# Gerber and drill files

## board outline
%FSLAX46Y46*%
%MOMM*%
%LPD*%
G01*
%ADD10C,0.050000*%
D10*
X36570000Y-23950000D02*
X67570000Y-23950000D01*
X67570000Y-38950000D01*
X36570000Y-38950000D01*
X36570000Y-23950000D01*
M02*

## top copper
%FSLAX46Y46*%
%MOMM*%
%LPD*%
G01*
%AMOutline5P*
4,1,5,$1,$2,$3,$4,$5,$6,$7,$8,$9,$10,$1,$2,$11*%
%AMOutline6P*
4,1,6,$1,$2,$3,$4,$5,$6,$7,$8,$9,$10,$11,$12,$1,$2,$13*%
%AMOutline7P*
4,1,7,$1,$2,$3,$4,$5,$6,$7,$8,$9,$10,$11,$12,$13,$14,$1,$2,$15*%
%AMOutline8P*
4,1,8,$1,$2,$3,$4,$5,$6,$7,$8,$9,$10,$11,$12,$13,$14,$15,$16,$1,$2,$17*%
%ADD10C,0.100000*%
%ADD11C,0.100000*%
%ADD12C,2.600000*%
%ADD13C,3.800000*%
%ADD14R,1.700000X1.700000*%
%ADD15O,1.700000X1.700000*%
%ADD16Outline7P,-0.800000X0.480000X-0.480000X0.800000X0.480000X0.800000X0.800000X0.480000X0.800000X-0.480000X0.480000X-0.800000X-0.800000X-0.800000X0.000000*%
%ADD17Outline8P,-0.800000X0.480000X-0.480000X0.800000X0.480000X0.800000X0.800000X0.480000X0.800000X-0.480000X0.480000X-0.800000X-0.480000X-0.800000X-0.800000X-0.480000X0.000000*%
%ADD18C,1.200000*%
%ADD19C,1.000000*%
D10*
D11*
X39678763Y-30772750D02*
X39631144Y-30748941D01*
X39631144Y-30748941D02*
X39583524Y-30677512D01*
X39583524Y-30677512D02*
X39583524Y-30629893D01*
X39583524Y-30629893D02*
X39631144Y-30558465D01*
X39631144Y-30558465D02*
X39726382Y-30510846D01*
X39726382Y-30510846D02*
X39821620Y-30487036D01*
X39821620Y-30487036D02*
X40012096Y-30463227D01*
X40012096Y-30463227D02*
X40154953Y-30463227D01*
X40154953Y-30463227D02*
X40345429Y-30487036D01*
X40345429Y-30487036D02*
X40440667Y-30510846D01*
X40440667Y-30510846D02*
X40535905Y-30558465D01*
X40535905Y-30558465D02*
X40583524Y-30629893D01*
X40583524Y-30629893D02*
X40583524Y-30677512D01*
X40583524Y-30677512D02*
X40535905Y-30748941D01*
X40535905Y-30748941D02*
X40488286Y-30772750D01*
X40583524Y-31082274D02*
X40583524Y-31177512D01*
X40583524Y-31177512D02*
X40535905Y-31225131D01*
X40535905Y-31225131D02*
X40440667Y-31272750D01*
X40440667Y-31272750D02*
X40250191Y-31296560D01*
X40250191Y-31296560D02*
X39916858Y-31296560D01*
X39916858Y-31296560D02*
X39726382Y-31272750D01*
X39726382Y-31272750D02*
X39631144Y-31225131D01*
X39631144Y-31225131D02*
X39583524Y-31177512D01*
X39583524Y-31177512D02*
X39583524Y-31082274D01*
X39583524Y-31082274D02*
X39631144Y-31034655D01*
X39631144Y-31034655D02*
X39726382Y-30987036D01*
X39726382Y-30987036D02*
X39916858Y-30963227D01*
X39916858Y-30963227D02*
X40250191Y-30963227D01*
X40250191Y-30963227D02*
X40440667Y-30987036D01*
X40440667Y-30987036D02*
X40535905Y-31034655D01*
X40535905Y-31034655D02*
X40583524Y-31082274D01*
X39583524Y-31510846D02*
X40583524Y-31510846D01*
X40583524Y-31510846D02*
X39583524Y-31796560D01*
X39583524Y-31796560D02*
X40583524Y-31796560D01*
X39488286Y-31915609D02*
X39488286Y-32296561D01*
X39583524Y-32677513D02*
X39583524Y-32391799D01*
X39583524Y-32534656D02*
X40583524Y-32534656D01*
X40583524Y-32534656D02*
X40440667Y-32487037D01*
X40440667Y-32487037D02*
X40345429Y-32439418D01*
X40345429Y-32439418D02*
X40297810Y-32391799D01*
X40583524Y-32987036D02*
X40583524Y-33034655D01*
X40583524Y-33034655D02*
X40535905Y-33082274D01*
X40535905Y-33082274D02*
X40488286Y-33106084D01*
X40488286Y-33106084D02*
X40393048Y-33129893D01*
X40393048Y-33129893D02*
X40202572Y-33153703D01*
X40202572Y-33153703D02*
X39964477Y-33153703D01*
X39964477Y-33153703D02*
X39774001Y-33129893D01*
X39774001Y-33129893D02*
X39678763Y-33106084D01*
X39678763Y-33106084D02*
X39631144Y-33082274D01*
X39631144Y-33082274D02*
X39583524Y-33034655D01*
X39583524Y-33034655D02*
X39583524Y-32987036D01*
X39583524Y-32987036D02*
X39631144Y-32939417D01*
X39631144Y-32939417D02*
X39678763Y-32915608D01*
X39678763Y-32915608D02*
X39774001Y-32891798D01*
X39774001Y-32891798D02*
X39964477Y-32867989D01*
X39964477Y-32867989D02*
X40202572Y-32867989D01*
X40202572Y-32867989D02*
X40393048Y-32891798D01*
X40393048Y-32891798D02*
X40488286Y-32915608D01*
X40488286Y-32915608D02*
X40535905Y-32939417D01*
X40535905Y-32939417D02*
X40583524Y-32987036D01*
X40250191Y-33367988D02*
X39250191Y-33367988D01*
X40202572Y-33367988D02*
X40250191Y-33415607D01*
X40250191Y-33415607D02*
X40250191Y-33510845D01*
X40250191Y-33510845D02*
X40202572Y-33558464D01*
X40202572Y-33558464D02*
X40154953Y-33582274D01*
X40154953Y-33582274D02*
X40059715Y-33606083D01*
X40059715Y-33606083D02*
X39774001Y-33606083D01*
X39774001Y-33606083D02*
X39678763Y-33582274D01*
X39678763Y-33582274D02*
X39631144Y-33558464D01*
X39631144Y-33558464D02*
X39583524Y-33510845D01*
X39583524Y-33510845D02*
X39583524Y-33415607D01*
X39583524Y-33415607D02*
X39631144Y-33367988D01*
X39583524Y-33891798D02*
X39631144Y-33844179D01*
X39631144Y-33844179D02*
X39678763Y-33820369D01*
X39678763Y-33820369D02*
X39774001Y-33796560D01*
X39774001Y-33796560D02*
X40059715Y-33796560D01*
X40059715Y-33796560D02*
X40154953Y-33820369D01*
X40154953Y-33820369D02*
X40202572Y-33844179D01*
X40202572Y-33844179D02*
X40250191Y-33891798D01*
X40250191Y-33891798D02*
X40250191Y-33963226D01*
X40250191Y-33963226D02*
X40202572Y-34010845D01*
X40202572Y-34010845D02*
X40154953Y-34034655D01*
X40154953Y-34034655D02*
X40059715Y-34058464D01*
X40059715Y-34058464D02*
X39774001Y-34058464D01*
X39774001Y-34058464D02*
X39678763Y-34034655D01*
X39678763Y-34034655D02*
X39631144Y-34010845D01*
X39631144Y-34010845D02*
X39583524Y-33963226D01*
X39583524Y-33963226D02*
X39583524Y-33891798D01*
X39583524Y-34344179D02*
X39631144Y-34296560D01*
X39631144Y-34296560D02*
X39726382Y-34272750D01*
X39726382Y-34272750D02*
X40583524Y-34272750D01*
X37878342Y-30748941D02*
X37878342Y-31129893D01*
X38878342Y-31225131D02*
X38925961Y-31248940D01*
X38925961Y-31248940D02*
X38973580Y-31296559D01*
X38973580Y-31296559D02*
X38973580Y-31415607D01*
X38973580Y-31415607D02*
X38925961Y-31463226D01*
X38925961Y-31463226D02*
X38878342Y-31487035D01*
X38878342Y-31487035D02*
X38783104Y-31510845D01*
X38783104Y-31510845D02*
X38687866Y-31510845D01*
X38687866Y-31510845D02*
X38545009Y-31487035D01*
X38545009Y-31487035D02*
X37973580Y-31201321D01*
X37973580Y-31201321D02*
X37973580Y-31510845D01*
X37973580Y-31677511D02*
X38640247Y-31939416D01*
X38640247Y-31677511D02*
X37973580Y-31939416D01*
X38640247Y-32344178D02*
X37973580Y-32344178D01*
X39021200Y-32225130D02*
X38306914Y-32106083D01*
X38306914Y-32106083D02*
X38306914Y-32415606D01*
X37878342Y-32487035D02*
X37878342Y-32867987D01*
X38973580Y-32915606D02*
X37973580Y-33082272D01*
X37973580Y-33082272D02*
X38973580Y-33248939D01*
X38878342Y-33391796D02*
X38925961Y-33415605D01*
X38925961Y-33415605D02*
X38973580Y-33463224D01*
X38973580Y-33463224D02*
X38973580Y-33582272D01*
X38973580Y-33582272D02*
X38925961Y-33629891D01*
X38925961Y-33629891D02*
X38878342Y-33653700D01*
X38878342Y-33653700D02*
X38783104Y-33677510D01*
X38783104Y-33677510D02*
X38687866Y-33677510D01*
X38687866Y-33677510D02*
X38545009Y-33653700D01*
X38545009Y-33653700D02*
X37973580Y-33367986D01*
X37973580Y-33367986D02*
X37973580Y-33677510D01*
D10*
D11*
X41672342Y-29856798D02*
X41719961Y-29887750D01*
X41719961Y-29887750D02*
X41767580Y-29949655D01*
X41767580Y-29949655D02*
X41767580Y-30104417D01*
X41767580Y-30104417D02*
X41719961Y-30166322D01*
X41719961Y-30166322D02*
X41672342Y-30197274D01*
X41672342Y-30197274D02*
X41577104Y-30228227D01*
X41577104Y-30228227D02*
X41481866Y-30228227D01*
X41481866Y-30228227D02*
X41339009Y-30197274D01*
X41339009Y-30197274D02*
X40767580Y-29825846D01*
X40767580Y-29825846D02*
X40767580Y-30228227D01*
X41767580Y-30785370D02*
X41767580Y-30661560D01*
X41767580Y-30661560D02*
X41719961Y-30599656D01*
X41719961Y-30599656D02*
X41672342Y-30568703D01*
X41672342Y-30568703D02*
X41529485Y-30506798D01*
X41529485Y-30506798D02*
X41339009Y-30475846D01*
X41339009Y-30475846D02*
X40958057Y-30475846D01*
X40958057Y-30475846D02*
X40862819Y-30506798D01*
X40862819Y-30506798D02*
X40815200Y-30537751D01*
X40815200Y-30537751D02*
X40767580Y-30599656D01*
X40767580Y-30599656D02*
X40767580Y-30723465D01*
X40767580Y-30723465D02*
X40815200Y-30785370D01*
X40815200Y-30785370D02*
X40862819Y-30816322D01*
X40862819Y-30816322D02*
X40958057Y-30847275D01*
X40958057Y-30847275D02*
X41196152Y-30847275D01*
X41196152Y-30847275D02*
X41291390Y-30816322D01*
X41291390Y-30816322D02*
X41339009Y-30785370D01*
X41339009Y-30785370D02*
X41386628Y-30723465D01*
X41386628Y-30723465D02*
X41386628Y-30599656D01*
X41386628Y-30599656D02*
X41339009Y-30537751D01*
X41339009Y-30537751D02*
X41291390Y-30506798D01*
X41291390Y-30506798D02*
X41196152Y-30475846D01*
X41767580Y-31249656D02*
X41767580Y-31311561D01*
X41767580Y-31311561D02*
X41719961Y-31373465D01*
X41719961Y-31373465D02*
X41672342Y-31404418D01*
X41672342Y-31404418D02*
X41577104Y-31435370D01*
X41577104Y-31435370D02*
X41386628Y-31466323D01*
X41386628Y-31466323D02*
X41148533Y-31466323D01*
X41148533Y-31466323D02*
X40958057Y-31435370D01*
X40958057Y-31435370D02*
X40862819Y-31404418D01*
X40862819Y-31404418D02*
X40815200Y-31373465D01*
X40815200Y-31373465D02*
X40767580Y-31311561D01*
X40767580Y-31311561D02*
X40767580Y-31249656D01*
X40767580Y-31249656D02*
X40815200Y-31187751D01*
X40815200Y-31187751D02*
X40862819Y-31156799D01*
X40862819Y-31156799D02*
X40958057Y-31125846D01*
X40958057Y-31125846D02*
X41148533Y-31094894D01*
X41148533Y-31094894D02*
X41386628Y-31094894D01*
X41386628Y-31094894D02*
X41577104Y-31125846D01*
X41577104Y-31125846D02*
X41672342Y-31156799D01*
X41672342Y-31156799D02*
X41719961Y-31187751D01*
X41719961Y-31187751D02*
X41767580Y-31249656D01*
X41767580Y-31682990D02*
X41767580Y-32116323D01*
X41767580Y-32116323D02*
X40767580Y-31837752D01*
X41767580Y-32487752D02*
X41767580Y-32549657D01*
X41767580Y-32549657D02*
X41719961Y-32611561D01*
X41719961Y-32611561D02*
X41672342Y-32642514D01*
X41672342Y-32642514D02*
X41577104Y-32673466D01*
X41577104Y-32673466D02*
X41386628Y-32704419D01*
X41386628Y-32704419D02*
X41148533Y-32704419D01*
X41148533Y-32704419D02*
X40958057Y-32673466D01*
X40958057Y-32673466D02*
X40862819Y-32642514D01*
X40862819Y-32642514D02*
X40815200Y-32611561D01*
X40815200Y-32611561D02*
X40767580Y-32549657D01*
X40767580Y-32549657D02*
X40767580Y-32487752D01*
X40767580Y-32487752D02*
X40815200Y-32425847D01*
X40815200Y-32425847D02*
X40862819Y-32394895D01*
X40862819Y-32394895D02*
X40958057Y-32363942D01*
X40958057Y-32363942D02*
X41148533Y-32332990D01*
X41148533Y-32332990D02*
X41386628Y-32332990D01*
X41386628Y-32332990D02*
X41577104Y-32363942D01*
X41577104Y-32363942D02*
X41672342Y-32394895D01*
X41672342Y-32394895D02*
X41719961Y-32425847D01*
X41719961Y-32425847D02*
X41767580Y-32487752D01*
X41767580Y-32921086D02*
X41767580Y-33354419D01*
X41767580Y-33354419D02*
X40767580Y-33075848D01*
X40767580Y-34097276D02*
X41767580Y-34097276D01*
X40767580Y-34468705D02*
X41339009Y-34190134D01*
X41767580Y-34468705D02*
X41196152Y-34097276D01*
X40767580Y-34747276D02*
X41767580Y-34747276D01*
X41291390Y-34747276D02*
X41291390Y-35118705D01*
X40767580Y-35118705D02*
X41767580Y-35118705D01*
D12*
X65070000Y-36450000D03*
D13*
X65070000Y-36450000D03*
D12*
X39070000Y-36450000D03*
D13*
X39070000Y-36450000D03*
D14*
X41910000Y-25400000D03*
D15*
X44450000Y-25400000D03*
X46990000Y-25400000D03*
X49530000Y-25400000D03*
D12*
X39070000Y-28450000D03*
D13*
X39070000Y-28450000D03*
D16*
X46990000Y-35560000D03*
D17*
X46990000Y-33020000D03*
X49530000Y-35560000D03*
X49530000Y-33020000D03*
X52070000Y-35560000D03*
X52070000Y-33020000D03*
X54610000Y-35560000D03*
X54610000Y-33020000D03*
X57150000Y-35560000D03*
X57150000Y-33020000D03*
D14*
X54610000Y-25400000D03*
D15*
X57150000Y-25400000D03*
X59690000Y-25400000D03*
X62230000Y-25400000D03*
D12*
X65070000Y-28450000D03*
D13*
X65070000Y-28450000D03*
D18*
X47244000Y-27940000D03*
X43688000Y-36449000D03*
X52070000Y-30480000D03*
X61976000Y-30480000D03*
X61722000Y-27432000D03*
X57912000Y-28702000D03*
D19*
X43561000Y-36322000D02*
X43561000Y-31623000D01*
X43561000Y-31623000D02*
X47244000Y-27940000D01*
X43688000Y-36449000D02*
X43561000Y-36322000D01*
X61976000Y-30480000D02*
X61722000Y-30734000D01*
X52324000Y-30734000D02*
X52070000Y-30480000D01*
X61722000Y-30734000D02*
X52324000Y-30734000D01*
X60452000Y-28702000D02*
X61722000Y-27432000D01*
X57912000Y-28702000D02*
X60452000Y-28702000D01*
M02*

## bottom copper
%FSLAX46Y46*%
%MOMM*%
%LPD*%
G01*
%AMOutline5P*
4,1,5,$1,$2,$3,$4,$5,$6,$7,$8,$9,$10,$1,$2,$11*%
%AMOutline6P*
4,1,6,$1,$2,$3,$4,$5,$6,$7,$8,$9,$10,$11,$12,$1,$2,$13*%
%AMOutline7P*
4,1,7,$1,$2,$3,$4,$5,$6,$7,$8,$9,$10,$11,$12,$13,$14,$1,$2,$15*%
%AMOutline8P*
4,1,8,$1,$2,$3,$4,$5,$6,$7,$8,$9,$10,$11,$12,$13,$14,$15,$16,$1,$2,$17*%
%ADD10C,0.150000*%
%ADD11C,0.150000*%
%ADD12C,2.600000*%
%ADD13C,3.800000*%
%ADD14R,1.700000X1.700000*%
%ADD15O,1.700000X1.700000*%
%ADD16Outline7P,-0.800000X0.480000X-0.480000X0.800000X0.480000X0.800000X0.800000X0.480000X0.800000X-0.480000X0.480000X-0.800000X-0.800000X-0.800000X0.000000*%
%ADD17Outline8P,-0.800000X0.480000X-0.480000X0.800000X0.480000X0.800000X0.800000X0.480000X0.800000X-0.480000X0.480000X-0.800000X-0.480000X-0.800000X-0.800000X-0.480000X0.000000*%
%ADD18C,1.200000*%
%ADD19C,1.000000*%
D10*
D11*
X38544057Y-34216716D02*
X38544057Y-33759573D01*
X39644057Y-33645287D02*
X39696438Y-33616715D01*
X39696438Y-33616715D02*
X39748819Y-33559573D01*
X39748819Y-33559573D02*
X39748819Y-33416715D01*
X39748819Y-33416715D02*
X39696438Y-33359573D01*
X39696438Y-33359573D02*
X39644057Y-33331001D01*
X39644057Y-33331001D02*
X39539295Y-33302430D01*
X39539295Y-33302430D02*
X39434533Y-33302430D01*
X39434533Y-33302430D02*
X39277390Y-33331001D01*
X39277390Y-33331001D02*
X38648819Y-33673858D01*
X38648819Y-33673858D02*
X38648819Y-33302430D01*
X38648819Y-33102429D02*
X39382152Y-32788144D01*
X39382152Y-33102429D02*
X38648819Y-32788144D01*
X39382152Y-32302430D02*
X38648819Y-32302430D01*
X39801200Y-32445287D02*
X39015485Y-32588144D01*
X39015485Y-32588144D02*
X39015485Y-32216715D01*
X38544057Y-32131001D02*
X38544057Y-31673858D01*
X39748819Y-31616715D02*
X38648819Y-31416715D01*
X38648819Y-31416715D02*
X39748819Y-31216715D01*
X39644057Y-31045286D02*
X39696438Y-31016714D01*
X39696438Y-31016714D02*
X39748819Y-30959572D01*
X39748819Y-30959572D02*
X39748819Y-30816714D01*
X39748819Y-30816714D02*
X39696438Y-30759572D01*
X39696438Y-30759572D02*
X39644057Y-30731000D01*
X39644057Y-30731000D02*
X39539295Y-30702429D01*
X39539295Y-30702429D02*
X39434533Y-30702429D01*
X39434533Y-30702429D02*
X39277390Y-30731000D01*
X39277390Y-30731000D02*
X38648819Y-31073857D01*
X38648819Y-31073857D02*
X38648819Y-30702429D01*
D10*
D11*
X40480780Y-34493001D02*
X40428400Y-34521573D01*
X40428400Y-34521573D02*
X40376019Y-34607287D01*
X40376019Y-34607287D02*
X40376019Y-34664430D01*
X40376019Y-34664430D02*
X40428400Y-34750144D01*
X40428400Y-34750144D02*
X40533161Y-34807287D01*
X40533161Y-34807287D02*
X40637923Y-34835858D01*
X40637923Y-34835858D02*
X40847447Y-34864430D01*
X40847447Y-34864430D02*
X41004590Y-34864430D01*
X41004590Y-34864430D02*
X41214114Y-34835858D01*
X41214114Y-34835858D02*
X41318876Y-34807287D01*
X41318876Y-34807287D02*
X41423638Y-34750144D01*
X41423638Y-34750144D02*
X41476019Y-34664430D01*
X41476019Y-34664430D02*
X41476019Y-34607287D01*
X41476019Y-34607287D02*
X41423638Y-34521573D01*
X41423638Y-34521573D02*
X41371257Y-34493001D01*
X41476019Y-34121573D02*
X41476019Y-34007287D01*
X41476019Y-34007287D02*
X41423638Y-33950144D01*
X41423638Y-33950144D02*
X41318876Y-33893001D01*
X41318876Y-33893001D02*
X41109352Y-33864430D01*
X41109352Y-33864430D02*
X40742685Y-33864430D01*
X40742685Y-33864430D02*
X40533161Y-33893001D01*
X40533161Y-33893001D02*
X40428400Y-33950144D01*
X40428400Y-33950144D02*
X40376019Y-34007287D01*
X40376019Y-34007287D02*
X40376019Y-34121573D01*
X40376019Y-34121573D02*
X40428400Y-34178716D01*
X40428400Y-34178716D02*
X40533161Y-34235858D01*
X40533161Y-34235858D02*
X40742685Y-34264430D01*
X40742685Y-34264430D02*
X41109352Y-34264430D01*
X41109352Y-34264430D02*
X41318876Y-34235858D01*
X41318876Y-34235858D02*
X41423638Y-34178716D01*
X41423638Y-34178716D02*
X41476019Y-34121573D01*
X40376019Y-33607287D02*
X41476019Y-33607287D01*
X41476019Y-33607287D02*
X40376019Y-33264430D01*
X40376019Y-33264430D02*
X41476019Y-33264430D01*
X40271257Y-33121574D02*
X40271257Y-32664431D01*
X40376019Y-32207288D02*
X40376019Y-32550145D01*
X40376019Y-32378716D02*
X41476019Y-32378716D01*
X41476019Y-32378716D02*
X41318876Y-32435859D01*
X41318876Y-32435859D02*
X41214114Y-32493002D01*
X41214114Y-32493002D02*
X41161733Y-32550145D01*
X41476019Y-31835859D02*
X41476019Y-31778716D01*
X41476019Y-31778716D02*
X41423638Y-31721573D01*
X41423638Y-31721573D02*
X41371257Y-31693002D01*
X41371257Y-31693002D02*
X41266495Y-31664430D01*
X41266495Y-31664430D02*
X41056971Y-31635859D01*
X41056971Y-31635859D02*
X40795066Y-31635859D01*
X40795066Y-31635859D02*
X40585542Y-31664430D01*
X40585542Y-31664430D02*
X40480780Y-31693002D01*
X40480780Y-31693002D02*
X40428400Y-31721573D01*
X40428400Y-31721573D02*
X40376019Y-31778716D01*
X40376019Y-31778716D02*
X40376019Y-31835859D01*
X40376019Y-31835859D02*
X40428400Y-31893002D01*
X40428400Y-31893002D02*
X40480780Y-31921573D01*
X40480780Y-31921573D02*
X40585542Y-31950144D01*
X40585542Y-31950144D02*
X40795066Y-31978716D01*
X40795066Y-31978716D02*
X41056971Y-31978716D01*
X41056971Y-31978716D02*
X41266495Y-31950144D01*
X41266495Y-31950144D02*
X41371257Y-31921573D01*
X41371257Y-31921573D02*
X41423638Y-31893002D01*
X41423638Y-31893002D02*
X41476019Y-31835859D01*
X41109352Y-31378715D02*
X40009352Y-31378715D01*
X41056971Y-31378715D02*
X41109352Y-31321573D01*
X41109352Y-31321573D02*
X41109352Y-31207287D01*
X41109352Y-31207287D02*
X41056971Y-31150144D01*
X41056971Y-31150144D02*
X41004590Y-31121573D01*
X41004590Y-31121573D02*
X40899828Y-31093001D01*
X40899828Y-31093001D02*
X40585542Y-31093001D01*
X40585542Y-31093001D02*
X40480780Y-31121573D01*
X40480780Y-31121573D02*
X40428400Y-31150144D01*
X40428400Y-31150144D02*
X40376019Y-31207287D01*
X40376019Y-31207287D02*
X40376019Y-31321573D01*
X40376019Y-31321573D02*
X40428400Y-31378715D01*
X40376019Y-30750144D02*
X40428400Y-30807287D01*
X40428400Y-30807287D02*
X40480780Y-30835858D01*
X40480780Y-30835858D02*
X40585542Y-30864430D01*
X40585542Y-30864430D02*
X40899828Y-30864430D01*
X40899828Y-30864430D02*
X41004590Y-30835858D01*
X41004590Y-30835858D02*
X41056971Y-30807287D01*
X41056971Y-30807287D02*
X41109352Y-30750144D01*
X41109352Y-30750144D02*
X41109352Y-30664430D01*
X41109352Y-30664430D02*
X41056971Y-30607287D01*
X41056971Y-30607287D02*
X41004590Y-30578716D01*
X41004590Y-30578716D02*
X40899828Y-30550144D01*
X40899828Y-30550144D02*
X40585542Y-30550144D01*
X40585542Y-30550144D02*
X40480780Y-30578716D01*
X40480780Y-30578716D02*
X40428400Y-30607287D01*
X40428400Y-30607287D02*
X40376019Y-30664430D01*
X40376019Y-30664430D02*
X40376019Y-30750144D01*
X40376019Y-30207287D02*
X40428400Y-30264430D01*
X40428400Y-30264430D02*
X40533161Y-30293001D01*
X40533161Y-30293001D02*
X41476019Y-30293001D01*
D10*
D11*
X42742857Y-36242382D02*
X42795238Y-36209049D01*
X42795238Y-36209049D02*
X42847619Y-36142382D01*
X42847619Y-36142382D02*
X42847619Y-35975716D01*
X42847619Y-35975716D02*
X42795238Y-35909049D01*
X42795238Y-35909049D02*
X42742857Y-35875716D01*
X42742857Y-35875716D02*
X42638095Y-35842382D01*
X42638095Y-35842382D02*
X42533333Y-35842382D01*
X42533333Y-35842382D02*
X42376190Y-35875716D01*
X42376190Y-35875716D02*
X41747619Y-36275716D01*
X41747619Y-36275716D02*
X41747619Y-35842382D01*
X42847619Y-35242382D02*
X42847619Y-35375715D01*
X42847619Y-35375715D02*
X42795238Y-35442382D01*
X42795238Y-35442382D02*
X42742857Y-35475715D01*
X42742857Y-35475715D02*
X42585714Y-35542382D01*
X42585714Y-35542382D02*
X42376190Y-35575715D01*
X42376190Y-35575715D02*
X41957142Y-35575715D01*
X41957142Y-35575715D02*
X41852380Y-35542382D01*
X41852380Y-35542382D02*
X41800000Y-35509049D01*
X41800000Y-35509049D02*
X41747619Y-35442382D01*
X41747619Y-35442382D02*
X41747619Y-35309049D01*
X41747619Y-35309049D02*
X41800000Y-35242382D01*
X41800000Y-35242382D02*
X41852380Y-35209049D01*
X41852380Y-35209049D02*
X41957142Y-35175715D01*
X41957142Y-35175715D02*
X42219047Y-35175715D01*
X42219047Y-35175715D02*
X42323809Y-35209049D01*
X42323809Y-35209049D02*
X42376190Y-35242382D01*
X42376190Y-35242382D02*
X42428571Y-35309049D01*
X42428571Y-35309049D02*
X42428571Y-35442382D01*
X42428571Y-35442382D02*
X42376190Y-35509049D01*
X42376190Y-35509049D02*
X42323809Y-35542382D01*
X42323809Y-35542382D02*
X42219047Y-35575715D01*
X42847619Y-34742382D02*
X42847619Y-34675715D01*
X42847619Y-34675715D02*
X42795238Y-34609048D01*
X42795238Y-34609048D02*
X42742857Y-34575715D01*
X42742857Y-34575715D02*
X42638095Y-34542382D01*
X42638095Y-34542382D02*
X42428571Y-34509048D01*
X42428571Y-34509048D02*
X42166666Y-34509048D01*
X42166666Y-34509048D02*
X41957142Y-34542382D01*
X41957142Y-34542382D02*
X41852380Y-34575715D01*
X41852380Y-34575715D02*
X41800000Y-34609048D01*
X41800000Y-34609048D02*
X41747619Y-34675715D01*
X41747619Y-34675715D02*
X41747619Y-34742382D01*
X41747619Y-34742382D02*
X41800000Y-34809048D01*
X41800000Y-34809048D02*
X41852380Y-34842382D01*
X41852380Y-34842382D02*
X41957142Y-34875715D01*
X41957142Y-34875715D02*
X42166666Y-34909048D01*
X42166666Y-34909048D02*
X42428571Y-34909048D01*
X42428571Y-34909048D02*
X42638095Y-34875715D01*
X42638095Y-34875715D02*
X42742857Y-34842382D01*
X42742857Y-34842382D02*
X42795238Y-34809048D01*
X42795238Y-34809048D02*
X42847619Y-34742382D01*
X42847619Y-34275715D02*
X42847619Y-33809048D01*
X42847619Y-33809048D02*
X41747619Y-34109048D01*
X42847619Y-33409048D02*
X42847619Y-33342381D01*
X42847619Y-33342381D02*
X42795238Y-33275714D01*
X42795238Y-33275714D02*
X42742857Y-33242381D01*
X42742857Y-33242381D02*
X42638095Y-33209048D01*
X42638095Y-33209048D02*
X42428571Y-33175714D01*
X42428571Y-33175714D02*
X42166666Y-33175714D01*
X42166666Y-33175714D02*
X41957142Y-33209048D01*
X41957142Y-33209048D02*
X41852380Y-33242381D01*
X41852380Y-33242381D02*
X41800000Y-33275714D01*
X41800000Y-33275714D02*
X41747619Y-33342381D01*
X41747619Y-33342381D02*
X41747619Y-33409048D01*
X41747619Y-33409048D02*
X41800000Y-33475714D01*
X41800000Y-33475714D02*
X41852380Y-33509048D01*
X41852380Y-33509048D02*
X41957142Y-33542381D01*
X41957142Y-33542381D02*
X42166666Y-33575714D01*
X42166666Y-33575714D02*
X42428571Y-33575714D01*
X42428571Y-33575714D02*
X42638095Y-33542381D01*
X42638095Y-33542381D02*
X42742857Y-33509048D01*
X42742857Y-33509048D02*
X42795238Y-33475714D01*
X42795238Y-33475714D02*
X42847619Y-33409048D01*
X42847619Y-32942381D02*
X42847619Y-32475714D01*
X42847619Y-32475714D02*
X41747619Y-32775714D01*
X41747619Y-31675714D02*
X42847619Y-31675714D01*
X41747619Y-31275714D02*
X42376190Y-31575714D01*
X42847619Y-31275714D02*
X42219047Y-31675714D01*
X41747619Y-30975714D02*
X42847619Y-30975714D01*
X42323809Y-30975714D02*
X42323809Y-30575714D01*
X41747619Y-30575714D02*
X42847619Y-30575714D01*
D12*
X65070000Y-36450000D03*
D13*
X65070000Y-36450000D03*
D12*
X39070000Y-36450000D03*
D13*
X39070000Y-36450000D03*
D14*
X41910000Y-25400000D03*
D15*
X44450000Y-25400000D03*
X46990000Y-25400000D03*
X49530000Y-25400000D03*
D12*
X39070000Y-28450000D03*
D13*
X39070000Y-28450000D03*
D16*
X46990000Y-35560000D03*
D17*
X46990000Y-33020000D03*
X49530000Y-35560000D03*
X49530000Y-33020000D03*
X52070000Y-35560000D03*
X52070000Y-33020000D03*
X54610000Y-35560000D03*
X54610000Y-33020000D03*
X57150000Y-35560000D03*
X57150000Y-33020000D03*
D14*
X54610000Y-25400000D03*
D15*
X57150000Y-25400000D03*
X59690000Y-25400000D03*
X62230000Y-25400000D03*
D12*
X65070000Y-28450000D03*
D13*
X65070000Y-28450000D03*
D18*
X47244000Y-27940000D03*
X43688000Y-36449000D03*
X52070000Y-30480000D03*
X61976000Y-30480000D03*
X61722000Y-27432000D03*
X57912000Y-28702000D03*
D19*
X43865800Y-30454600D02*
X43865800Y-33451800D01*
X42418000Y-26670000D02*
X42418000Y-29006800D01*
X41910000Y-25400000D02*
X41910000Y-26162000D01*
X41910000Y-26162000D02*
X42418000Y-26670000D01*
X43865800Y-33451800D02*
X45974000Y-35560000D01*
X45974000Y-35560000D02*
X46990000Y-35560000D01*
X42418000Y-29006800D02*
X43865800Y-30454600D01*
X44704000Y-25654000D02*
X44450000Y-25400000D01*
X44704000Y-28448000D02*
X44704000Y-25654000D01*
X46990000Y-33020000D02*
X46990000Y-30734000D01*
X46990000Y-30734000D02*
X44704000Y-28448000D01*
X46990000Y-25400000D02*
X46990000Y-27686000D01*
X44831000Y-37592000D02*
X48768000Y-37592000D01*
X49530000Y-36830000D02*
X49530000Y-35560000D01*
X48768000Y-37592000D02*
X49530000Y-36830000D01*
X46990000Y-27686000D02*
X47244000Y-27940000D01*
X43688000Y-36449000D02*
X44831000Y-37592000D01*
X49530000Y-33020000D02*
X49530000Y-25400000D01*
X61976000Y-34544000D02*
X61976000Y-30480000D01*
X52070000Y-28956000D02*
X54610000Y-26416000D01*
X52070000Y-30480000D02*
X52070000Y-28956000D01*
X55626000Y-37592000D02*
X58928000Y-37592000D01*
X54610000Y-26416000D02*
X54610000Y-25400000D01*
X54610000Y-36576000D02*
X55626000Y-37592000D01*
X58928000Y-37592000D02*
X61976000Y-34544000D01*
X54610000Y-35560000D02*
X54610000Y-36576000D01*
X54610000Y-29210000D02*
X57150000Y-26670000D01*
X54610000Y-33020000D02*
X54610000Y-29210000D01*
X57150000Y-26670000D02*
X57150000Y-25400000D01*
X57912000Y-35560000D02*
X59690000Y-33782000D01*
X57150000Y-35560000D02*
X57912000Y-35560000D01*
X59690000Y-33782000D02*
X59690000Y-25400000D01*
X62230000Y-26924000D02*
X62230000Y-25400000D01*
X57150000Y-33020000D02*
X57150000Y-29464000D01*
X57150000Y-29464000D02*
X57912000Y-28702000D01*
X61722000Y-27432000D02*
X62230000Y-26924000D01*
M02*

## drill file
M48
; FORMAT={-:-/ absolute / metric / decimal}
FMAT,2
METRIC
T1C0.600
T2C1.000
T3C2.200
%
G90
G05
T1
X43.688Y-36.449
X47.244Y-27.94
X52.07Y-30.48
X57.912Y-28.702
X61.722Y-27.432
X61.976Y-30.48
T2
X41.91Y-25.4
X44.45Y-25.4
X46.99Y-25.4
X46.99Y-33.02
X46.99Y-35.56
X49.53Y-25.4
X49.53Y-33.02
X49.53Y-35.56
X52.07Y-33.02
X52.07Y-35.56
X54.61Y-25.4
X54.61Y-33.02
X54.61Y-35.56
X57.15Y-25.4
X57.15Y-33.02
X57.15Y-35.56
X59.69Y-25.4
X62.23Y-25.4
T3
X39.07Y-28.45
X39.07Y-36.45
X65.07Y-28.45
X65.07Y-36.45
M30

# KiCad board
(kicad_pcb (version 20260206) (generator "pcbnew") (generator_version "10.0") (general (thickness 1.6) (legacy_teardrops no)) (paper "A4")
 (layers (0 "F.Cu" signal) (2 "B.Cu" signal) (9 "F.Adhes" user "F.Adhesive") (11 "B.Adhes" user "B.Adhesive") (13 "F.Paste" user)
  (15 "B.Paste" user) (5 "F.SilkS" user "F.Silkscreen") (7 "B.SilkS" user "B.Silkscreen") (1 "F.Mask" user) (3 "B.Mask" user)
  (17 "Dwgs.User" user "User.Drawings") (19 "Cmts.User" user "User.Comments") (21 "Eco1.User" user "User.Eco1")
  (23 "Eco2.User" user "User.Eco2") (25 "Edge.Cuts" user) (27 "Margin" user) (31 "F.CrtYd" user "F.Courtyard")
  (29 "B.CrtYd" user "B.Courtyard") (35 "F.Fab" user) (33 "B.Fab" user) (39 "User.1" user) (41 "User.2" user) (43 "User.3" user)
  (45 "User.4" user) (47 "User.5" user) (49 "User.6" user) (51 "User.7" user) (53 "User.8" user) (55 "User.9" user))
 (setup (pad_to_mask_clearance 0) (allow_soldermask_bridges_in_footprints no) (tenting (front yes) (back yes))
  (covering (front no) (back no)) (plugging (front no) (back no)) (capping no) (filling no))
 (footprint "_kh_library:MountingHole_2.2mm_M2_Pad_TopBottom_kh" (layer "F.Cu") (at 65.07 36.45)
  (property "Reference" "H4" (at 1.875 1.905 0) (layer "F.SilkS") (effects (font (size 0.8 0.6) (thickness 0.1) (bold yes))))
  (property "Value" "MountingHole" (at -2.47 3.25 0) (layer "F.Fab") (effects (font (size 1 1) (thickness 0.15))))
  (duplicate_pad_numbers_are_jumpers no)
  (pad "1" thru_hole circle (at 0 0) (size 2.6 2.6) (drill 2.2) (layers "*.Cu" "*.Mask") (remove_unused_layers no))
  (pad "1" connect circle (at 0 0) (size 3.8 3.8) (layers "F.Cu" "F.Mask"))
  (pad "1" connect circle (at 0 0) (size 3.8 3.8) (layers "B.Cu" "B.Mask")))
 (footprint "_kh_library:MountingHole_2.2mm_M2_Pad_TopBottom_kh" (layer "F.Cu") (at 39.07 36.45)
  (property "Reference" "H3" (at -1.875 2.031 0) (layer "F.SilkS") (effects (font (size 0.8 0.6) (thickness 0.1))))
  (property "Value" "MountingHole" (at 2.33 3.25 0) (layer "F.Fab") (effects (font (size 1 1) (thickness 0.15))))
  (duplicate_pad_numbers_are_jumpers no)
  (pad "1" thru_hole circle (at 0 0) (size 2.6 2.6) (drill 2.2) (layers "*.Cu" "*.Mask") (remove_unused_layers no))
  (pad "1" connect circle (at 0 0) (size 3.8 3.8) (layers "F.Cu" "F.Mask"))
  (pad "1" connect circle (at 0 0) (size 3.8 3.8) (layers "B.Cu" "B.Mask")))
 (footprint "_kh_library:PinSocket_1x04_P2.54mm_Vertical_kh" (layer "F.Cu") (at 41.91 25.4 90)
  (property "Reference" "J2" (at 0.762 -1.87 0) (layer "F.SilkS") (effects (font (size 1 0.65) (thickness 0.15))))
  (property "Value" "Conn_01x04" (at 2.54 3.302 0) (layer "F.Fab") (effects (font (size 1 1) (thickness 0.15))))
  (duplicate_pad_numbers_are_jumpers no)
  (pad "1" thru_hole rect (at 0 0 90) (size 1.7 1.7) (drill 1) (layers "*.Cu" "*.Mask") (remove_unused_layers no) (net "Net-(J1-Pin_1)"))
  (pad "2" thru_hole oval (at 0 2.54 90) (size 1.7 1.7) (drill 1) (layers "*.Cu" "*.Mask") (remove_unused_layers no) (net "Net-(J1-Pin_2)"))
  (pad "3" thru_hole oval (at 0 5.08 90) (size 1.7 1.7) (drill 1) (layers "*.Cu" "*.Mask") (remove_unused_layers no) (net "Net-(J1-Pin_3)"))
  (pad "4" thru_hole oval (at 0 7.62 90) (size 1.7 1.7) (drill 1) (layers "*.Cu" "*.Mask") (remove_unused_layers no) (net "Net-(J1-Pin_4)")))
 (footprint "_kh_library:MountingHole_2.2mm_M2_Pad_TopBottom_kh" (layer "F.Cu") (at 39.07 28.45)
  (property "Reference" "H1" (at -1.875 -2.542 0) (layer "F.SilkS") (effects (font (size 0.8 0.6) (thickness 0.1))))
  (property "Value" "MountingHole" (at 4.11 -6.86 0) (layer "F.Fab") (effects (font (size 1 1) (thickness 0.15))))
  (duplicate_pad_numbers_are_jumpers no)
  (pad "1" thru_hole circle (at 0 0) (size 2.6 2.6) (drill 2.2) (layers "*.Cu" "*.Mask") (remove_unused_layers no))
  (pad "1" connect circle (at 0 0) (size 3.8 3.8) (layers "F.Cu" "F.Mask"))
  (pad "1" connect circle (at 0 0) (size 3.8 3.8) (layers "B.Cu" "B.Mask")))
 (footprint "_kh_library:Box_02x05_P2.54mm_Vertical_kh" (layer "F.Cu") (at 46.99 35.56)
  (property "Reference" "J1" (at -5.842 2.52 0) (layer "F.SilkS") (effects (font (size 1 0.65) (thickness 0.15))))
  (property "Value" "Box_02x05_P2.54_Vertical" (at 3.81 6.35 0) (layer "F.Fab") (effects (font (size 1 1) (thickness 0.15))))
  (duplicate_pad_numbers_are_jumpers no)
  (pad "1" thru_hole roundrect (at 0 0) (size 1.6 1.6) (drill 1) (layers "*.Cu" "*.Mask") (remove_unused_layers no) (roundrect_rratio 0)
   (chamfer_ratio 0.2) (chamfer top_left top_right bottom_right) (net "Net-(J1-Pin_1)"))
  (pad "2" thru_hole roundrect (at 0 -2.54) (size 1.6 1.6) (drill 1) (layers "*.Cu" "*.Mask") (remove_unused_layers no) (roundrect_rratio 0)
   (chamfer_ratio 0.2) (chamfer top_left top_right bottom_left bottom_right) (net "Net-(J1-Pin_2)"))
  (pad "3" thru_hole roundrect (at 2.54 0) (size 1.6 1.6) (drill 1) (layers "*.Cu" "*.Mask") (remove_unused_layers no) (roundrect_rratio 0)
   (chamfer_ratio 0.2) (chamfer top_left top_right bottom_left bottom_right) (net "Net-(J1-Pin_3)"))
  (pad "4" thru_hole roundrect (at 2.54 -2.54) (size 1.6 1.6) (drill 1) (layers "*.Cu" "*.Mask") (remove_unused_layers no)
   (roundrect_rratio 0) (chamfer_ratio 0.2) (chamfer top_left top_right bottom_left bottom_right) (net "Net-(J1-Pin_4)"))
  (pad "5" thru_hole roundrect (at 5.08 0) (size 1.6 1.6) (drill 1) (layers "*.Cu" "*.Mask") (remove_unused_layers no) (roundrect_rratio 0)
   (chamfer_ratio 0.2) (chamfer top_left top_right bottom_left bottom_right) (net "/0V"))
  (pad "6" thru_hole roundrect (at 5.08 -2.54) (size 1.6 1.6) (drill 1) (layers "*.Cu" "*.Mask") (remove_unused_layers no)
   (roundrect_rratio 0) (chamfer_ratio 0.2) (chamfer top_left top_right bottom_left bottom_right) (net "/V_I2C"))
  (pad "7" thru_hole roundrect (at 7.62 0) (size 1.6 1.6) (drill 1) (layers "*.Cu" "*.Mask") (remove_unused_layers no) (roundrect_rratio 0)
   (chamfer_ratio 0.2) (chamfer top_left top_right bottom_left bottom_right) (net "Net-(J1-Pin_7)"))
  (pad "8" thru_hole roundrect (at 7.62 -2.54) (size 1.6 1.6) (drill 1) (layers "*.Cu" "*.Mask") (remove_unused_layers no)
   (roundrect_rratio 0) (chamfer_ratio 0.2) (chamfer top_left top_right bottom_left bottom_right) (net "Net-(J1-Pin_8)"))
  (pad "9" thru_hole roundrect (at 10.16 0) (size 1.6 1.6) (drill 1) (layers "*.Cu" "*.Mask") (remove_unused_layers no) (roundrect_rratio 0)
   (chamfer_ratio 0.2) (chamfer top_left top_right bottom_left bottom_right) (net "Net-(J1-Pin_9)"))
  (pad "10" thru_hole roundrect (at 10.16 -2.54) (size 1.6 1.6) (drill 1) (layers "*.Cu" "*.Mask") (remove_unused_layers no)
   (roundrect_rratio 0) (chamfer_ratio 0.2) (chamfer top_left top_right bottom_left bottom_right) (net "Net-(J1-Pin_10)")))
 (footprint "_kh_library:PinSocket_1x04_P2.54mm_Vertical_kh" (layer "F.Cu") (at 54.61 25.4 90)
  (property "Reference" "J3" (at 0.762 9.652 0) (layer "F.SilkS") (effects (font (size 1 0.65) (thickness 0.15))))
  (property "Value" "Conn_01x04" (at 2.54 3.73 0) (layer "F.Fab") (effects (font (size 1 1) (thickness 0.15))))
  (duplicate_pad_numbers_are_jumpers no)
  (pad "1" thru_hole rect (at 0 0 90) (size 1.7 1.7) (drill 1) (layers "*.Cu" "*.Mask") (remove_unused_layers no) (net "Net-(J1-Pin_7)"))
  (pad "2" thru_hole oval (at 0 2.54 90) (size 1.7 1.7) (drill 1) (layers "*.Cu" "*.Mask") (remove_unused_layers no) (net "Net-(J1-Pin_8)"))
  (pad "3" thru_hole oval (at 0 5.08 90) (size 1.7 1.7) (drill 1) (layers "*.Cu" "*.Mask") (remove_unused_layers no) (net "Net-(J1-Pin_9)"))
  (pad "4" thru_hole oval (at 0 7.62 90) (size 1.7 1.7) (drill 1) (layers "*.Cu" "*.Mask") (remove_unused_layers no) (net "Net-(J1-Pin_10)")))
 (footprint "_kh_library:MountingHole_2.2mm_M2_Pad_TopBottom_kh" (layer "F.Cu") (at 65.07 28.45)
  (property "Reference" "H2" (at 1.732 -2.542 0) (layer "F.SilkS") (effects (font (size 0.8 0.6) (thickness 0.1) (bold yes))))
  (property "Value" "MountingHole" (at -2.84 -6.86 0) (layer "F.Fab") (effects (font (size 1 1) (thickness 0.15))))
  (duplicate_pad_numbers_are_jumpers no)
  (pad "1" thru_hole circle (at 0 0) (size 2.6 2.6) (drill 2.2) (layers "*.Cu" "*.Mask") (remove_unused_layers no))
  (pad "1" connect circle (at 0 0) (size 3.8 3.8) (layers "F.Cu" "F.Mask"))
  (pad "1" connect circle (at 0 0) (size 3.8 3.8) (layers "B.Cu" "B.Mask")))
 (gr_rect (start 36.57 23.95) (end 67.57 38.95) (stroke (width 0.05) (type default)) (fill no) (layer "Edge.Cuts"))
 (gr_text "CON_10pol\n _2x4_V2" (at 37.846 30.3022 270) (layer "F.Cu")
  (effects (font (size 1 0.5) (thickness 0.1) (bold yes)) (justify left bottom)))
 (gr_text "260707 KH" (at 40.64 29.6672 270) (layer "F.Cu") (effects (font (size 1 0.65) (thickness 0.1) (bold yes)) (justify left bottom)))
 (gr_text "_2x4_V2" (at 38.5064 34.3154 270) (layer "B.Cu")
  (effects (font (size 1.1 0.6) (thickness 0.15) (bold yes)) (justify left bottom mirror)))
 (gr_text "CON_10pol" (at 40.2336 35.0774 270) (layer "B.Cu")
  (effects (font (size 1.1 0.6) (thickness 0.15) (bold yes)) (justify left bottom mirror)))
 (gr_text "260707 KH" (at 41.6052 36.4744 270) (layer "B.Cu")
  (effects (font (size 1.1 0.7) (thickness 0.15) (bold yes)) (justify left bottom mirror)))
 (segment (start 43.8658 30.4546) (end 43.8658 33.4518) (width 1) (layer "B.Cu") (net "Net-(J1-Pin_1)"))
 (segment (start 42.418 26.67) (end 42.418 29.0068) (width 1) (layer "B.Cu") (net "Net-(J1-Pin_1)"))
 (segment (start 41.91 25.4) (end 41.91 26.162) (width 1) (layer "B.Cu") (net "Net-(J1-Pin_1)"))
 (segment (start 41.91 26.162) (end 42.418 26.67) (width 1) (layer "B.Cu") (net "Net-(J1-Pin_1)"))
 (segment (start 43.8658 33.4518) (end 45.974 35.56) (width 1) (layer "B.Cu") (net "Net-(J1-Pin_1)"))
 (segment (start 45.974 35.56) (end 46.99 35.56) (width 1) (layer "B.Cu") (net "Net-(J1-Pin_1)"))
 (segment (start 42.418 29.0068) (end 43.8658 30.4546) (width 1) (layer "B.Cu") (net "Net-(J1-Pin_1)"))
 (segment (start 44.704 25.654) (end 44.45 25.4) (width 1) (layer "B.Cu") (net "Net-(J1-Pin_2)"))
 (segment (start 44.704 28.448) (end 44.704 25.654) (width 1) (layer "B.Cu") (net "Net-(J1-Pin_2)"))
 (segment (start 46.99 33.02) (end 46.99 30.734) (width 1) (layer "B.Cu") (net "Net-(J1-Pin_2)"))
 (segment (start 46.99 30.734) (end 44.704 28.448) (width 1) (layer "B.Cu") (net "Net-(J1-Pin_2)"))
 (segment (start 43.561 36.322) (end 43.561 31.623) (width 1) (layer "F.Cu") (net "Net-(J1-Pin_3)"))
 (segment (start 43.561 31.623) (end 47.244 27.94) (width 1) (layer "F.Cu") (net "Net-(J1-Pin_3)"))
 (segment (start 43.688 36.449) (end 43.561 36.322) (width 1) (layer "F.Cu") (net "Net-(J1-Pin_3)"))
 (via (at 47.244 27.94) (size 1.2) (drill 0.6) (layers "F.Cu" "B.Cu") (capping no) (covering (front no) (back no))
  (plugging (front no) (back no)) (filling no) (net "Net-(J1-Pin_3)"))
 (via (at 43.688 36.449) (size 1.2) (drill 0.6) (layers "F.Cu" "B.Cu") (capping no) (covering (front no) (back no))
  (plugging (front no) (back no)) (filling no) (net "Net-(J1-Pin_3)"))
 (segment (start 46.99 25.4) (end 46.99 27.686) (width 1) (layer "B.Cu") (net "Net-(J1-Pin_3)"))
 (segment (start 44.831 37.592) (end 48.768 37.592) (width 1) (layer "B.Cu") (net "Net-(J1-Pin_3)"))
 (segment (start 49.53 36.83) (end 49.53 35.56) (width 1) (layer "B.Cu") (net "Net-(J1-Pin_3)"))
 (segment (start 48.768 37.592) (end 49.53 36.83) (width 1) (layer "B.Cu") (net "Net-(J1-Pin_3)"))
 (segment (start 46.99 27.686) (end 47.244 27.94) (width 1) (layer "B.Cu") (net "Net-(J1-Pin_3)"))
 (segment (start 43.688 36.449) (end 44.831 37.592) (width 1) (layer "B.Cu") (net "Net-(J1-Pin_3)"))
 (segment (start 49.53 33.02) (end 49.53 25.4) (width 1) (layer "B.Cu") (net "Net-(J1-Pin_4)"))
 (segment (start 61.976 30.48) (end 61.722 30.734) (width 1) (layer "F.Cu") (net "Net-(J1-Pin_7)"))
 (segment (start 52.324 30.734) (end 52.07 30.48) (width 1) (layer "F.Cu") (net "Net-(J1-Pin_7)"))
 (segment (start 61.722 30.734) (end 52.324 30.734) (width 1) (layer "F.Cu") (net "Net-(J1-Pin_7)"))
 (via (at 52.07 30.48) (size 1.2) (drill 0.6) (layers "F.Cu" "B.Cu") (capping no) (covering (front no) (back no))
  (plugging (front no) (back no)) (filling no) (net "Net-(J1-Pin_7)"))
 (via (at 61.976 30.48) (size 1.2) (drill 0.6) (layers "F.Cu" "B.Cu") (capping no) (covering (front no) (back no))
  (plugging (front no) (back no)) (filling no) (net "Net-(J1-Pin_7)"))
 (segment (start 61.976 34.544) (end 61.976 30.48) (width 1) (layer "B.Cu") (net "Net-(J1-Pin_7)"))
 (segment (start 52.07 28.956) (end 54.61 26.416) (width 1) (layer "B.Cu") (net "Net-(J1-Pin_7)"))
 (segment (start 52.07 30.48) (end 52.07 28.956) (width 1) (layer "B.Cu") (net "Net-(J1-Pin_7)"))
 (segment (start 55.626 37.592) (end 58.928 37.592) (width 1) (layer "B.Cu") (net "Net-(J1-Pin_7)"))
 (segment (start 54.61 26.416) (end 54.61 25.4) (width 1) (layer "B.Cu") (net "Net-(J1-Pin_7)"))
 (segment (start 54.61 36.576) (end 55.626 37.592) (width 1) (layer "B.Cu") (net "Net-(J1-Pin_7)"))
 (segment (start 58.928 37.592) (end 61.976 34.544) (width 1) (layer "B.Cu") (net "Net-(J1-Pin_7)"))
 (segment (start 54.61 35.56) (end 54.61 36.576) (width 1) (layer "B.Cu") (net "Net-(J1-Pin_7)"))
 (segment (start 54.61 29.21) (end 57.15 26.67) (width 1) (layer "B.Cu") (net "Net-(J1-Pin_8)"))
 (segment (start 54.61 33.02) (end 54.61 29.21) (width 1) (layer "B.Cu") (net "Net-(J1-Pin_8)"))
 (segment (start 57.15 26.67) (end 57.15 25.4) (width 1) (layer "B.Cu") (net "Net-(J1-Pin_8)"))
 (segment (start 57.912 35.56) (end 59.69 33.782) (width 1) (layer "B.Cu") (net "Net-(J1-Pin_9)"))
 (segment (start 57.15 35.56) (end 57.912 35.56) (width 1) (layer "B.Cu") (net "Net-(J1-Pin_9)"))
 (segment (start 59.69 33.782) (end 59.69 25.4) (width 1) (layer "B.Cu") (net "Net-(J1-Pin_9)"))
 (segment (start 60.452 28.702) (end 61.722 27.432) (width 1) (layer "F.Cu") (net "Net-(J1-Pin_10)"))
 (segment (start 57.912 28.702) (end 60.452 28.702) (width 1) (layer "F.Cu") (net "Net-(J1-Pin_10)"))
 (via (at 61.722 27.432) (size 1.2) (drill 0.6) (layers "F.Cu" "B.Cu") (capping no) (covering (front no) (back no))
  (plugging (front no) (back no)) (filling no) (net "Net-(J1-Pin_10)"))
 (via (at 57.912 28.702) (size 1.2) (drill 0.6) (layers "F.Cu" "B.Cu") (capping no) (covering (front no) (back no))
  (plugging (front no) (back no)) (filling no) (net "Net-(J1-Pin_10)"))
 (segment (start 62.23 26.924) (end 62.23 25.4) (width 1) (layer "B.Cu") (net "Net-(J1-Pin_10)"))
 (segment (start 57.15 33.02) (end 57.15 29.464) (width 1) (layer "B.Cu") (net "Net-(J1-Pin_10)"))
 (segment (start 57.15 29.464) (end 57.912 28.702) (width 1) (layer "B.Cu") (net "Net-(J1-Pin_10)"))
 (segment (start 61.722 27.432) (end 62.23 26.924) (width 1) (layer "B.Cu") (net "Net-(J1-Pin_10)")))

